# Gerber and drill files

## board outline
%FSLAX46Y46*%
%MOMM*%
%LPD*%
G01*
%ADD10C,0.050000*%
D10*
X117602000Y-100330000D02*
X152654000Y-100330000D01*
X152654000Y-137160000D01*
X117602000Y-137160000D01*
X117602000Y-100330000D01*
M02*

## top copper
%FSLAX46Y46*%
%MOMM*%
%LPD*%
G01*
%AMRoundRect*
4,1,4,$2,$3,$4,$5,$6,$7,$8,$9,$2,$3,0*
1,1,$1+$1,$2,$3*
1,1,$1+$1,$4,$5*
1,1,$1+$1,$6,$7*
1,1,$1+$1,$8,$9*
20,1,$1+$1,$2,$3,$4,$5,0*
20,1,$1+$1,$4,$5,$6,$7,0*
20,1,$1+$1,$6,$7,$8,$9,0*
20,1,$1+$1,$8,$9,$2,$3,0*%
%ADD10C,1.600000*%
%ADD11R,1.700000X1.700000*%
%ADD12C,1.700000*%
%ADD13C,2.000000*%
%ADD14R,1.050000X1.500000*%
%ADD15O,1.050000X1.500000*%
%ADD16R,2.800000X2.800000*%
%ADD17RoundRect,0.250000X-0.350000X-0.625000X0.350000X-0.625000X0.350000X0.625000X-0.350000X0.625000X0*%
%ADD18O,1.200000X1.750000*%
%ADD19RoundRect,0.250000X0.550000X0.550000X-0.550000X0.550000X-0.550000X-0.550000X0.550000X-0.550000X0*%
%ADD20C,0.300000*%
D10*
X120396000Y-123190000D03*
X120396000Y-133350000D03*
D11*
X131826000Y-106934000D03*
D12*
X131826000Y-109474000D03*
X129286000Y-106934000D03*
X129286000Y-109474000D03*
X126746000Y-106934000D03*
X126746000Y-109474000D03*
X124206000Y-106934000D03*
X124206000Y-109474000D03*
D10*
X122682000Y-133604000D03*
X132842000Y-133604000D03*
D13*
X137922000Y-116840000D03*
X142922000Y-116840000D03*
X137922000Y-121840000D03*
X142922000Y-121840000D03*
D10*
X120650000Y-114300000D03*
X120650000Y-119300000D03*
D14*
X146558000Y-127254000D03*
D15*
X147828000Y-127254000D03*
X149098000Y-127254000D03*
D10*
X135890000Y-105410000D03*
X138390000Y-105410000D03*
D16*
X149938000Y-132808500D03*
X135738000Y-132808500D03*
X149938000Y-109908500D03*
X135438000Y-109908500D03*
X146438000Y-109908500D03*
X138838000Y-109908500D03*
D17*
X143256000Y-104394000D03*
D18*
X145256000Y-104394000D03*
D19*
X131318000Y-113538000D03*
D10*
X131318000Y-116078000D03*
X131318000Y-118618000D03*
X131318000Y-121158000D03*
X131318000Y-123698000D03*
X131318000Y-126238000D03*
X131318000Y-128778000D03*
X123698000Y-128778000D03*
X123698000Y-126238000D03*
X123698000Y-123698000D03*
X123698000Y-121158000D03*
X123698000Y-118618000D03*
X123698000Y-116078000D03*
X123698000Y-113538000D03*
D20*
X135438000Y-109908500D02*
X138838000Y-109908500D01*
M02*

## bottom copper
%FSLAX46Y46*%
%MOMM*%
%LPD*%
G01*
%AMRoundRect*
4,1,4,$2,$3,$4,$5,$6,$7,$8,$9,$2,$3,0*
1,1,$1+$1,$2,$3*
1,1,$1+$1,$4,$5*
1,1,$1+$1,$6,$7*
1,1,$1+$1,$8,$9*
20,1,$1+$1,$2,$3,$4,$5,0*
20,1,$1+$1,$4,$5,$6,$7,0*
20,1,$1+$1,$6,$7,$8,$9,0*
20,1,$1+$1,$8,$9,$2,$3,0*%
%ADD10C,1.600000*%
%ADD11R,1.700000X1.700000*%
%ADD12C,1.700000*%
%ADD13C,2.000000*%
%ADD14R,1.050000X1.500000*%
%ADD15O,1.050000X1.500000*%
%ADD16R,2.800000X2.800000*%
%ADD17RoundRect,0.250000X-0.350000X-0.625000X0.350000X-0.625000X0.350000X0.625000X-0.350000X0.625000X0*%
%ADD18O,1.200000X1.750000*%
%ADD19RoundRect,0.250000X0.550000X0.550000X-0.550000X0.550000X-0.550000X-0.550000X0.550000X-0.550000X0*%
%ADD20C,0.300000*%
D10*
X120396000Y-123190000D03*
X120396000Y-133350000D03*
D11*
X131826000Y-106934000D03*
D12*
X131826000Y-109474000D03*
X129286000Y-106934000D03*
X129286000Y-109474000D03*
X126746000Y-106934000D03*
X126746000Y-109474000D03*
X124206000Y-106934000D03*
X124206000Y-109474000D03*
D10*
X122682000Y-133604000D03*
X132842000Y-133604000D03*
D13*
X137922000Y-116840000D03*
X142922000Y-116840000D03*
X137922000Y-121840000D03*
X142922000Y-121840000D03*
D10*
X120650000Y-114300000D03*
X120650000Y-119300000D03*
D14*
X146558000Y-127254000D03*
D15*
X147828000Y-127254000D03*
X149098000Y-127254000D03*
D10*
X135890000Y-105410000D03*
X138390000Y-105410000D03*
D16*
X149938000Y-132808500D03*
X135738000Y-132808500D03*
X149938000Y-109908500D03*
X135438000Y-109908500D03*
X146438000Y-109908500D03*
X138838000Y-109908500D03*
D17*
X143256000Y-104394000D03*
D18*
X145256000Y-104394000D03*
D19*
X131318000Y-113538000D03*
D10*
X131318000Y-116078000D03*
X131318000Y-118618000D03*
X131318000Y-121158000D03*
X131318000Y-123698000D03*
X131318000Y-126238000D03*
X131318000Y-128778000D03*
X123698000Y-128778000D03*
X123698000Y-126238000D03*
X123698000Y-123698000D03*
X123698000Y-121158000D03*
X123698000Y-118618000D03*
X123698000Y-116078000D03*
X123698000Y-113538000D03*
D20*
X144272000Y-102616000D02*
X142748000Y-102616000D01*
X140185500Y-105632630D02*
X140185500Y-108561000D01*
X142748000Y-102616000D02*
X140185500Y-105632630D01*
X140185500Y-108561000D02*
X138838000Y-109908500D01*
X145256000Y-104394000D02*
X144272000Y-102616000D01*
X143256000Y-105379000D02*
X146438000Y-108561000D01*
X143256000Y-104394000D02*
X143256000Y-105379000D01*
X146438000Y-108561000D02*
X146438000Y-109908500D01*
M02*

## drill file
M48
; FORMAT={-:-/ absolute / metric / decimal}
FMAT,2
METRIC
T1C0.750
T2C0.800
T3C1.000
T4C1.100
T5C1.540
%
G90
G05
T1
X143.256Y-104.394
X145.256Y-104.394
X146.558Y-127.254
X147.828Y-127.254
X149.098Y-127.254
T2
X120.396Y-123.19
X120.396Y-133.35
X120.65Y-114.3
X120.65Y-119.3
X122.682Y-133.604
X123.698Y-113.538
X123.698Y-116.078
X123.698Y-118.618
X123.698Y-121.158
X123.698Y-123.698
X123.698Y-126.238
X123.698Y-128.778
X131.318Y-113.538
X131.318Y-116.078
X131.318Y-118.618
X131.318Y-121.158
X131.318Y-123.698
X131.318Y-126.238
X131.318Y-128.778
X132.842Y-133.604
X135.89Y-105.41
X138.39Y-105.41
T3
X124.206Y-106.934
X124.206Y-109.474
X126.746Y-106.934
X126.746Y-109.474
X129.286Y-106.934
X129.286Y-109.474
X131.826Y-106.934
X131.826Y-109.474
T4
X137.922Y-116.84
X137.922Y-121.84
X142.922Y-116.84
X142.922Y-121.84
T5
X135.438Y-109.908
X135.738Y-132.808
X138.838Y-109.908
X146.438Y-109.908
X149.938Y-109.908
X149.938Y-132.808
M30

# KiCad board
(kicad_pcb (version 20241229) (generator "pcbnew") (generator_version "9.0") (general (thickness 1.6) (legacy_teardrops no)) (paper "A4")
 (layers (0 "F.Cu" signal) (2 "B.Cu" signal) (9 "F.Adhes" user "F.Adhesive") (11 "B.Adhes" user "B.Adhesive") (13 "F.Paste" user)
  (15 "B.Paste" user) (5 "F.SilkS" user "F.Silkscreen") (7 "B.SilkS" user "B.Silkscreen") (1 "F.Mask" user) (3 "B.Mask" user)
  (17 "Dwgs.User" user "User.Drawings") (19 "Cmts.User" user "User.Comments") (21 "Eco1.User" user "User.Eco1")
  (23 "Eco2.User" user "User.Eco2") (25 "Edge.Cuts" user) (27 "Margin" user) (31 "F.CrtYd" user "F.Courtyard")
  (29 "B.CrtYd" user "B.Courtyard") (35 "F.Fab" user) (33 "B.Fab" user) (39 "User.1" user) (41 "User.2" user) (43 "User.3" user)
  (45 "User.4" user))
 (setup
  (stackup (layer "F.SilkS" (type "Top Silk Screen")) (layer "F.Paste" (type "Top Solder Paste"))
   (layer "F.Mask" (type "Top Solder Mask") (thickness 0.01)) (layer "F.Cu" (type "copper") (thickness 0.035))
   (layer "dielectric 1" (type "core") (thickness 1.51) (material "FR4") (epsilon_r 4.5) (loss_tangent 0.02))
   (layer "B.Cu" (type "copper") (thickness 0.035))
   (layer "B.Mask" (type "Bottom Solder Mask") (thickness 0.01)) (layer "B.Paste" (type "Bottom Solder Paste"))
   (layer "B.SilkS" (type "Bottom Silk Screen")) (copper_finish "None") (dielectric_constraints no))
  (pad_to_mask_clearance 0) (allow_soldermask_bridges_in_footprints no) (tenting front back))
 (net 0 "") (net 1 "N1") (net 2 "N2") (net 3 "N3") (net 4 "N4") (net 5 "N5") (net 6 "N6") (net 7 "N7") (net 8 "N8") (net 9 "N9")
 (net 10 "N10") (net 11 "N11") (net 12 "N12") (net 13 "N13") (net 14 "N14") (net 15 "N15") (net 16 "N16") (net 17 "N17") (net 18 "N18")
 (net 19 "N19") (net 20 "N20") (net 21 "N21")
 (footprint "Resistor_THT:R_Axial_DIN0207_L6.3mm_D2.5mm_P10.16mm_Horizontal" (layer "F.Cu") (at 120.396 123.19 -90)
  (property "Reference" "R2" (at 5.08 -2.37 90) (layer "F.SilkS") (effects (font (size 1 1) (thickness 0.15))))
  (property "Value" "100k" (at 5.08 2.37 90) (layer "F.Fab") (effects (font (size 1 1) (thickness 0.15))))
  (pad "1" thru_hole circle (at 0 0 270) (size 1.6 1.6) (drill 0.8) (layers "*.Cu" "*.Mask") (remove_unused_layers no) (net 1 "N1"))
  (pad "2" thru_hole circle (at 10.16 0 270) (size 1.6 1.6) (drill 0.8) (layers "*.Cu" "*.Mask") (remove_unused_layers no) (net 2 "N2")))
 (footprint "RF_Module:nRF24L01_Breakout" (layer "F.Cu") (at 131.826 106.934 -90)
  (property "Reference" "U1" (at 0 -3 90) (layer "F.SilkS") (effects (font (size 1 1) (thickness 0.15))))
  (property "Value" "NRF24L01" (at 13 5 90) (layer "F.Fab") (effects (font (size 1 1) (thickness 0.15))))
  (pad "1" thru_hole rect (at 0 0 270) (size 1.7 1.7) (drill 1) (layers "*.Cu" "*.Mask") (remove_unused_layers no) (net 2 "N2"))
  (pad "2" thru_hole circle (at 2.54 0 270) (size 1.7 1.7) (drill 1) (layers "*.Cu" "*.Mask") (remove_unused_layers no) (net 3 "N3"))
  (pad "3" thru_hole circle (at 0 2.54 270) (size 1.7 1.7) (drill 1) (layers "*.Cu" "*.Mask") (remove_unused_layers no) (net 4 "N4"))
  (pad "4" thru_hole circle (at 2.54 2.54 270) (size 1.7 1.7) (drill 1) (layers "*.Cu" "*.Mask") (remove_unused_layers no) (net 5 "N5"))
  (pad "5" thru_hole circle (at 0 5.08 270) (size 1.7 1.7) (drill 1) (layers "*.Cu" "*.Mask") (remove_unused_layers no) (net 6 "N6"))
  (pad "6" thru_hole circle (at 2.54 5.08 270) (size 1.7 1.7) (drill 1) (layers "*.Cu" "*.Mask") (remove_unused_layers no) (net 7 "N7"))
  (pad "7" thru_hole circle (at 0 7.62 270) (size 1.7 1.7) (drill 1) (layers "*.Cu" "*.Mask") (remove_unused_layers no) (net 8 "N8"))
  (pad "8" thru_hole circle (at 2.54 7.62 270) (size 1.7 1.7) (drill 1) (layers "*.Cu" "*.Mask") (remove_unused_layers no) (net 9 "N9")))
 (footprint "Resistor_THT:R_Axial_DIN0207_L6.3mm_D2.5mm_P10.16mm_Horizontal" (layer "F.Cu") (at 122.682 133.604)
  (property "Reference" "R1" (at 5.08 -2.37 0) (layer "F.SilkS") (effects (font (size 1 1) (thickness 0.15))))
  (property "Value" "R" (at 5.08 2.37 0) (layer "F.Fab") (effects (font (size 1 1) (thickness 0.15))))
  (pad "1" thru_hole circle (at 0 0) (size 1.6 1.6) (drill 0.8) (layers "*.Cu" "*.Mask") (remove_unused_layers no) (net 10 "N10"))
  (pad "2" thru_hole circle (at 10.16 0) (size 1.6 1.6) (drill 0.8) (layers "*.Cu" "*.Mask") (remove_unused_layers no) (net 1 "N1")))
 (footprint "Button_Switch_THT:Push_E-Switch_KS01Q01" (layer "F.Cu") (at 137.922 116.84)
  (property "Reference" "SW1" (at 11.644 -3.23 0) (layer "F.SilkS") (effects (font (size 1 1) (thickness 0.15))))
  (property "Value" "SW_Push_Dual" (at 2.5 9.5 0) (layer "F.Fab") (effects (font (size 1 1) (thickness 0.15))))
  (pad "1" thru_hole circle (at 0 0) (size 2 2) (drill 1.1) (layers "*.Cu" "*.Mask") (remove_unused_layers no) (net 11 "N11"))
  (pad "2" thru_hole circle (at 5 0) (size 2 2) (drill 1.1) (layers "*.Cu" "*.Mask") (remove_unused_layers no) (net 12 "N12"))
  (pad "3" thru_hole circle (at 0 5) (size 2 2) (drill 1.1) (layers "*.Cu" "*.Mask") (remove_unused_layers no) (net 2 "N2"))
  (pad "4" thru_hole circle (at 5 5) (size 2 2) (drill 1.1) (layers "*.Cu" "*.Mask") (remove_unused_layers no) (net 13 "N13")))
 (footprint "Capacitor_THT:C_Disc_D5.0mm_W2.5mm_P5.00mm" (layer "F.Cu") (at 120.65 114.3 -90)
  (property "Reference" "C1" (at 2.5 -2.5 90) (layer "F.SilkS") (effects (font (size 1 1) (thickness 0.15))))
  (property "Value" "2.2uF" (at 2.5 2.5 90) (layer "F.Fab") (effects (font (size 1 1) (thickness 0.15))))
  (pad "1" thru_hole circle (at 0 0 270) (size 1.6 1.6) (drill 0.8) (layers "*.Cu" "*.Mask") (remove_unused_layers no) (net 2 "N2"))
  (pad "2" thru_hole circle (at 5 0 270) (size 1.6 1.6) (drill 0.8) (layers "*.Cu" "*.Mask") (remove_unused_layers no) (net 3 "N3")))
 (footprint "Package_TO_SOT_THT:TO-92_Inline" (layer "F.Cu") (at 146.558 127.254)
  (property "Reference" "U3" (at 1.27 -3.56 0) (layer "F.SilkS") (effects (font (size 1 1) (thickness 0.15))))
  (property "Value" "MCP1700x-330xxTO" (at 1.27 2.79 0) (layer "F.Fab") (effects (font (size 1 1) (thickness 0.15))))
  (pad "1" thru_hole rect (at 0 0) (size 1.05 1.5) (drill 0.75) (layers "*.Cu" "*.Mask") (remove_unused_layers no) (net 2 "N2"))
  (pad "2" thru_hole oval (at 1.27 0) (size 1.05 1.5) (drill 0.75) (layers "*.Cu" "*.Mask") (remove_unused_layers no) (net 10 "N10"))
  (pad "3" thru_hole oval (at 2.54 0) (size 1.05 1.5) (drill 0.75) (layers "*.Cu" "*.Mask") (remove_unused_layers no) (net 3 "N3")))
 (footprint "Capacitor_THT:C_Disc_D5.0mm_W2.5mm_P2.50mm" (layer "F.Cu") (at 135.89 105.41)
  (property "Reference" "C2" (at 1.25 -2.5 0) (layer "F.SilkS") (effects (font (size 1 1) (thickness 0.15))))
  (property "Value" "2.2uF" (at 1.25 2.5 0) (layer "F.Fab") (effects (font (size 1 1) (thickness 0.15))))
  (pad "1" thru_hole circle (at 0 0) (size 1.6 1.6) (drill 0.8) (layers "*.Cu" "*.Mask") (remove_unused_layers no) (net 2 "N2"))
  (pad "2" thru_hole circle (at 2.5 0) (size 1.6 1.6) (drill 0.8) (layers "*.Cu" "*.Mask") (remove_unused_layers no) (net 10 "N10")))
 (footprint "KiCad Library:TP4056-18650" (layer "B.Cu") (at 151.638 134.5085 90)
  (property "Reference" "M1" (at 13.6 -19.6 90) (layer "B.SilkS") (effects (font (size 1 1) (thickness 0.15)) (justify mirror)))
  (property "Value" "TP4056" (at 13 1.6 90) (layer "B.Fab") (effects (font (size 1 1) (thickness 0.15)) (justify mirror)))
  (pad "1" thru_hole rect (at 1.7 -1.7 90) (size 2.8 2.8) (drill 1.54) (layers "*.Cu" "*.Mask") (remove_unused_layers no) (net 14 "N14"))
  (pad "2" thru_hole rect (at 1.7 -15.9 90) (size 2.8 2.8) (drill 1.54) (layers "*.Cu" "*.Mask") (remove_unused_layers no) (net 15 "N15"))
  (pad "3" thru_hole rect (at 24.6 -1.7 90) (size 2.8 2.8) (drill 1.54) (layers "*.Cu" "*.Mask") (remove_unused_layers no) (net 10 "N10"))
  (pad "4" thru_hole rect (at 24.6 -16.2 90) (size 2.8 2.8) (drill 1.54) (layers "*.Cu" "*.Mask") (remove_unused_layers no) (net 2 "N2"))
  (pad "5" thru_hole rect (at 24.6 -5.2 90) (size 2.8 2.8) (drill 1.54) (layers "*.Cu" "*.Mask") (remove_unused_layers no) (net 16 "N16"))
  (pad "6" thru_hole rect (at 24.6 -12.8 90) (size 2.8 2.8) (drill 1.54) (layers "*.Cu" "*.Mask") (remove_unused_layers no) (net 2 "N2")))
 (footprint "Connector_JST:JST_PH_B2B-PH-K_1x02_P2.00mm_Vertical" (layer "B.Cu") (at 143.256 104.394)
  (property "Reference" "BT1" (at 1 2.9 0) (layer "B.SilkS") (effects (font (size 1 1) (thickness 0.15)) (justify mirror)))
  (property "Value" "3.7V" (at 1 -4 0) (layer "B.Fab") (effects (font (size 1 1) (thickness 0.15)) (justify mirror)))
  (pad "1" thru_hole roundrect (at 0 0) (size 1.2 1.75) (drill 0.75) (layers "*.Cu" "*.Mask") (remove_unused_layers no)
   (roundrect_rratio 0.208333) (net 16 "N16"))
  (pad "2" thru_hole oval (at 2 0) (size 1.2 1.75) (drill 0.75) (layers "*.Cu" "*.Mask") (remove_unused_layers no) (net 2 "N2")))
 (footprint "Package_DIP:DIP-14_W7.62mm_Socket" (layer "B.Cu") (at 131.318 113.538 180)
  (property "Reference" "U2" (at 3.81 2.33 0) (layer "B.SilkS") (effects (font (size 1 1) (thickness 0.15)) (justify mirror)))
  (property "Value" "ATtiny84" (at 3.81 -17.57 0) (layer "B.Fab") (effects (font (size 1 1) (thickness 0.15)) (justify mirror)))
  (pad "1" thru_hole roundrect (at 0 0 180) (size 1.6 1.6) (drill 0.8) (layers "*.Cu" "*.Mask") (remove_unused_layers no)
   (roundrect_rratio 0.15625) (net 10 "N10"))
  (pad "2" thru_hole circle (at 0 -2.54 180) (size 1.6 1.6) (drill 0.8) (layers "*.Cu" "*.Mask") (remove_unused_layers no) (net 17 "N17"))
  (pad "3" thru_hole circle (at 0 -5.08 180) (size 1.6 1.6) (drill 0.8) (layers "*.Cu" "*.Mask") (remove_unused_layers no) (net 4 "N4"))
  (pad "4" thru_hole circle (at 0 -7.62 180) (size 1.6 1.6) (drill 0.8) (layers "*.Cu" "*.Mask") (remove_unused_layers no) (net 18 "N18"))
  (pad "5" thru_hole circle (at 0 -10.16 180) (size 1.6 1.6) (drill 0.8) (layers "*.Cu" "*.Mask") (remove_unused_layers no) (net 5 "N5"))
  (pad "6" thru_hole circle (at 0 -12.7 180) (size 1.6 1.6) (drill 0.8) (layers "*.Cu" "*.Mask") (remove_unused_layers no) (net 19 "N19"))
  (pad "7" thru_hole circle (at 0 -15.24 180) (size 1.6 1.6) (drill 0.8) (layers "*.Cu" "*.Mask") (remove_unused_layers no) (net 8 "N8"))
  (pad "8" thru_hole circle (at 7.62 -15.24 180) (size 1.6 1.6) (drill 0.8) (layers "*.Cu" "*.Mask") (remove_unused_layers no) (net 7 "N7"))
  (pad "9" thru_hole circle (at 7.62 -12.7 180) (size 1.6 1.6) (drill 0.8) (layers "*.Cu" "*.Mask") (remove_unused_layers no) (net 6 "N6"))
  (pad "10" thru_hole circle (at 7.62 -10.16 180) (size 1.6 1.6) (drill 0.8) (layers "*.Cu" "*.Mask") (remove_unused_layers no)
   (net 13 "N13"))
  (pad "11" thru_hole circle (at 7.62 -7.62 180) (size 1.6 1.6) (drill 0.8) (layers "*.Cu" "*.Mask") (remove_unused_layers no)
   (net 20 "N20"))
  (pad "12" thru_hole circle (at 7.62 -5.08 180) (size 1.6 1.6) (drill 0.8) (layers "*.Cu" "*.Mask") (remove_unused_layers no)
   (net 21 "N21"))
  (pad "13" thru_hole circle (at 7.62 -2.54 180) (size 1.6 1.6) (drill 0.8) (layers "*.Cu" "*.Mask") (remove_unused_layers no) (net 1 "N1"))
  (pad "14" thru_hole circle (at 7.62 0 180) (size 1.6 1.6) (drill 0.8) (layers "*.Cu" "*.Mask") (remove_unused_layers no) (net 2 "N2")))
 (gr_rect (start 117.602 100.33) (end 152.654 137.16) (stroke (width 0.05) (type default)) (fill no) (layer "Edge.Cuts"))
 (segment (start 135.438 109.9085) (end 138.838 109.9085) (width 0.3) (layer "F.Cu") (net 2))
 (segment (start 144.272 102.616) (end 142.748 102.616) (width 0.3) (layer "B.Cu") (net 2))
 (segment (start 140.1855 105.63263) (end 140.1855 108.561) (width 0.3) (layer "B.Cu") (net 2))
 (segment (start 142.748 102.616) (end 140.1855 105.63263) (width 0.3) (layer "B.Cu") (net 2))
 (segment (start 140.1855 108.561) (end 138.838 109.9085) (width 0.3) (layer "B.Cu") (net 2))
 (segment (start 145.256 104.394) (end 144.272 102.616) (width 0.3) (layer "B.Cu") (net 2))
 (segment (start 143.256 105.379) (end 146.438 108.561) (width 0.3) (layer "B.Cu") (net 16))
 (segment (start 143.256 104.394) (end 143.256 105.379) (width 0.3) (layer "B.Cu") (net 16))
 (segment (start 146.438 108.561) (end 146.438 109.9085) (width 0.3) (layer "B.Cu") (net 16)))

